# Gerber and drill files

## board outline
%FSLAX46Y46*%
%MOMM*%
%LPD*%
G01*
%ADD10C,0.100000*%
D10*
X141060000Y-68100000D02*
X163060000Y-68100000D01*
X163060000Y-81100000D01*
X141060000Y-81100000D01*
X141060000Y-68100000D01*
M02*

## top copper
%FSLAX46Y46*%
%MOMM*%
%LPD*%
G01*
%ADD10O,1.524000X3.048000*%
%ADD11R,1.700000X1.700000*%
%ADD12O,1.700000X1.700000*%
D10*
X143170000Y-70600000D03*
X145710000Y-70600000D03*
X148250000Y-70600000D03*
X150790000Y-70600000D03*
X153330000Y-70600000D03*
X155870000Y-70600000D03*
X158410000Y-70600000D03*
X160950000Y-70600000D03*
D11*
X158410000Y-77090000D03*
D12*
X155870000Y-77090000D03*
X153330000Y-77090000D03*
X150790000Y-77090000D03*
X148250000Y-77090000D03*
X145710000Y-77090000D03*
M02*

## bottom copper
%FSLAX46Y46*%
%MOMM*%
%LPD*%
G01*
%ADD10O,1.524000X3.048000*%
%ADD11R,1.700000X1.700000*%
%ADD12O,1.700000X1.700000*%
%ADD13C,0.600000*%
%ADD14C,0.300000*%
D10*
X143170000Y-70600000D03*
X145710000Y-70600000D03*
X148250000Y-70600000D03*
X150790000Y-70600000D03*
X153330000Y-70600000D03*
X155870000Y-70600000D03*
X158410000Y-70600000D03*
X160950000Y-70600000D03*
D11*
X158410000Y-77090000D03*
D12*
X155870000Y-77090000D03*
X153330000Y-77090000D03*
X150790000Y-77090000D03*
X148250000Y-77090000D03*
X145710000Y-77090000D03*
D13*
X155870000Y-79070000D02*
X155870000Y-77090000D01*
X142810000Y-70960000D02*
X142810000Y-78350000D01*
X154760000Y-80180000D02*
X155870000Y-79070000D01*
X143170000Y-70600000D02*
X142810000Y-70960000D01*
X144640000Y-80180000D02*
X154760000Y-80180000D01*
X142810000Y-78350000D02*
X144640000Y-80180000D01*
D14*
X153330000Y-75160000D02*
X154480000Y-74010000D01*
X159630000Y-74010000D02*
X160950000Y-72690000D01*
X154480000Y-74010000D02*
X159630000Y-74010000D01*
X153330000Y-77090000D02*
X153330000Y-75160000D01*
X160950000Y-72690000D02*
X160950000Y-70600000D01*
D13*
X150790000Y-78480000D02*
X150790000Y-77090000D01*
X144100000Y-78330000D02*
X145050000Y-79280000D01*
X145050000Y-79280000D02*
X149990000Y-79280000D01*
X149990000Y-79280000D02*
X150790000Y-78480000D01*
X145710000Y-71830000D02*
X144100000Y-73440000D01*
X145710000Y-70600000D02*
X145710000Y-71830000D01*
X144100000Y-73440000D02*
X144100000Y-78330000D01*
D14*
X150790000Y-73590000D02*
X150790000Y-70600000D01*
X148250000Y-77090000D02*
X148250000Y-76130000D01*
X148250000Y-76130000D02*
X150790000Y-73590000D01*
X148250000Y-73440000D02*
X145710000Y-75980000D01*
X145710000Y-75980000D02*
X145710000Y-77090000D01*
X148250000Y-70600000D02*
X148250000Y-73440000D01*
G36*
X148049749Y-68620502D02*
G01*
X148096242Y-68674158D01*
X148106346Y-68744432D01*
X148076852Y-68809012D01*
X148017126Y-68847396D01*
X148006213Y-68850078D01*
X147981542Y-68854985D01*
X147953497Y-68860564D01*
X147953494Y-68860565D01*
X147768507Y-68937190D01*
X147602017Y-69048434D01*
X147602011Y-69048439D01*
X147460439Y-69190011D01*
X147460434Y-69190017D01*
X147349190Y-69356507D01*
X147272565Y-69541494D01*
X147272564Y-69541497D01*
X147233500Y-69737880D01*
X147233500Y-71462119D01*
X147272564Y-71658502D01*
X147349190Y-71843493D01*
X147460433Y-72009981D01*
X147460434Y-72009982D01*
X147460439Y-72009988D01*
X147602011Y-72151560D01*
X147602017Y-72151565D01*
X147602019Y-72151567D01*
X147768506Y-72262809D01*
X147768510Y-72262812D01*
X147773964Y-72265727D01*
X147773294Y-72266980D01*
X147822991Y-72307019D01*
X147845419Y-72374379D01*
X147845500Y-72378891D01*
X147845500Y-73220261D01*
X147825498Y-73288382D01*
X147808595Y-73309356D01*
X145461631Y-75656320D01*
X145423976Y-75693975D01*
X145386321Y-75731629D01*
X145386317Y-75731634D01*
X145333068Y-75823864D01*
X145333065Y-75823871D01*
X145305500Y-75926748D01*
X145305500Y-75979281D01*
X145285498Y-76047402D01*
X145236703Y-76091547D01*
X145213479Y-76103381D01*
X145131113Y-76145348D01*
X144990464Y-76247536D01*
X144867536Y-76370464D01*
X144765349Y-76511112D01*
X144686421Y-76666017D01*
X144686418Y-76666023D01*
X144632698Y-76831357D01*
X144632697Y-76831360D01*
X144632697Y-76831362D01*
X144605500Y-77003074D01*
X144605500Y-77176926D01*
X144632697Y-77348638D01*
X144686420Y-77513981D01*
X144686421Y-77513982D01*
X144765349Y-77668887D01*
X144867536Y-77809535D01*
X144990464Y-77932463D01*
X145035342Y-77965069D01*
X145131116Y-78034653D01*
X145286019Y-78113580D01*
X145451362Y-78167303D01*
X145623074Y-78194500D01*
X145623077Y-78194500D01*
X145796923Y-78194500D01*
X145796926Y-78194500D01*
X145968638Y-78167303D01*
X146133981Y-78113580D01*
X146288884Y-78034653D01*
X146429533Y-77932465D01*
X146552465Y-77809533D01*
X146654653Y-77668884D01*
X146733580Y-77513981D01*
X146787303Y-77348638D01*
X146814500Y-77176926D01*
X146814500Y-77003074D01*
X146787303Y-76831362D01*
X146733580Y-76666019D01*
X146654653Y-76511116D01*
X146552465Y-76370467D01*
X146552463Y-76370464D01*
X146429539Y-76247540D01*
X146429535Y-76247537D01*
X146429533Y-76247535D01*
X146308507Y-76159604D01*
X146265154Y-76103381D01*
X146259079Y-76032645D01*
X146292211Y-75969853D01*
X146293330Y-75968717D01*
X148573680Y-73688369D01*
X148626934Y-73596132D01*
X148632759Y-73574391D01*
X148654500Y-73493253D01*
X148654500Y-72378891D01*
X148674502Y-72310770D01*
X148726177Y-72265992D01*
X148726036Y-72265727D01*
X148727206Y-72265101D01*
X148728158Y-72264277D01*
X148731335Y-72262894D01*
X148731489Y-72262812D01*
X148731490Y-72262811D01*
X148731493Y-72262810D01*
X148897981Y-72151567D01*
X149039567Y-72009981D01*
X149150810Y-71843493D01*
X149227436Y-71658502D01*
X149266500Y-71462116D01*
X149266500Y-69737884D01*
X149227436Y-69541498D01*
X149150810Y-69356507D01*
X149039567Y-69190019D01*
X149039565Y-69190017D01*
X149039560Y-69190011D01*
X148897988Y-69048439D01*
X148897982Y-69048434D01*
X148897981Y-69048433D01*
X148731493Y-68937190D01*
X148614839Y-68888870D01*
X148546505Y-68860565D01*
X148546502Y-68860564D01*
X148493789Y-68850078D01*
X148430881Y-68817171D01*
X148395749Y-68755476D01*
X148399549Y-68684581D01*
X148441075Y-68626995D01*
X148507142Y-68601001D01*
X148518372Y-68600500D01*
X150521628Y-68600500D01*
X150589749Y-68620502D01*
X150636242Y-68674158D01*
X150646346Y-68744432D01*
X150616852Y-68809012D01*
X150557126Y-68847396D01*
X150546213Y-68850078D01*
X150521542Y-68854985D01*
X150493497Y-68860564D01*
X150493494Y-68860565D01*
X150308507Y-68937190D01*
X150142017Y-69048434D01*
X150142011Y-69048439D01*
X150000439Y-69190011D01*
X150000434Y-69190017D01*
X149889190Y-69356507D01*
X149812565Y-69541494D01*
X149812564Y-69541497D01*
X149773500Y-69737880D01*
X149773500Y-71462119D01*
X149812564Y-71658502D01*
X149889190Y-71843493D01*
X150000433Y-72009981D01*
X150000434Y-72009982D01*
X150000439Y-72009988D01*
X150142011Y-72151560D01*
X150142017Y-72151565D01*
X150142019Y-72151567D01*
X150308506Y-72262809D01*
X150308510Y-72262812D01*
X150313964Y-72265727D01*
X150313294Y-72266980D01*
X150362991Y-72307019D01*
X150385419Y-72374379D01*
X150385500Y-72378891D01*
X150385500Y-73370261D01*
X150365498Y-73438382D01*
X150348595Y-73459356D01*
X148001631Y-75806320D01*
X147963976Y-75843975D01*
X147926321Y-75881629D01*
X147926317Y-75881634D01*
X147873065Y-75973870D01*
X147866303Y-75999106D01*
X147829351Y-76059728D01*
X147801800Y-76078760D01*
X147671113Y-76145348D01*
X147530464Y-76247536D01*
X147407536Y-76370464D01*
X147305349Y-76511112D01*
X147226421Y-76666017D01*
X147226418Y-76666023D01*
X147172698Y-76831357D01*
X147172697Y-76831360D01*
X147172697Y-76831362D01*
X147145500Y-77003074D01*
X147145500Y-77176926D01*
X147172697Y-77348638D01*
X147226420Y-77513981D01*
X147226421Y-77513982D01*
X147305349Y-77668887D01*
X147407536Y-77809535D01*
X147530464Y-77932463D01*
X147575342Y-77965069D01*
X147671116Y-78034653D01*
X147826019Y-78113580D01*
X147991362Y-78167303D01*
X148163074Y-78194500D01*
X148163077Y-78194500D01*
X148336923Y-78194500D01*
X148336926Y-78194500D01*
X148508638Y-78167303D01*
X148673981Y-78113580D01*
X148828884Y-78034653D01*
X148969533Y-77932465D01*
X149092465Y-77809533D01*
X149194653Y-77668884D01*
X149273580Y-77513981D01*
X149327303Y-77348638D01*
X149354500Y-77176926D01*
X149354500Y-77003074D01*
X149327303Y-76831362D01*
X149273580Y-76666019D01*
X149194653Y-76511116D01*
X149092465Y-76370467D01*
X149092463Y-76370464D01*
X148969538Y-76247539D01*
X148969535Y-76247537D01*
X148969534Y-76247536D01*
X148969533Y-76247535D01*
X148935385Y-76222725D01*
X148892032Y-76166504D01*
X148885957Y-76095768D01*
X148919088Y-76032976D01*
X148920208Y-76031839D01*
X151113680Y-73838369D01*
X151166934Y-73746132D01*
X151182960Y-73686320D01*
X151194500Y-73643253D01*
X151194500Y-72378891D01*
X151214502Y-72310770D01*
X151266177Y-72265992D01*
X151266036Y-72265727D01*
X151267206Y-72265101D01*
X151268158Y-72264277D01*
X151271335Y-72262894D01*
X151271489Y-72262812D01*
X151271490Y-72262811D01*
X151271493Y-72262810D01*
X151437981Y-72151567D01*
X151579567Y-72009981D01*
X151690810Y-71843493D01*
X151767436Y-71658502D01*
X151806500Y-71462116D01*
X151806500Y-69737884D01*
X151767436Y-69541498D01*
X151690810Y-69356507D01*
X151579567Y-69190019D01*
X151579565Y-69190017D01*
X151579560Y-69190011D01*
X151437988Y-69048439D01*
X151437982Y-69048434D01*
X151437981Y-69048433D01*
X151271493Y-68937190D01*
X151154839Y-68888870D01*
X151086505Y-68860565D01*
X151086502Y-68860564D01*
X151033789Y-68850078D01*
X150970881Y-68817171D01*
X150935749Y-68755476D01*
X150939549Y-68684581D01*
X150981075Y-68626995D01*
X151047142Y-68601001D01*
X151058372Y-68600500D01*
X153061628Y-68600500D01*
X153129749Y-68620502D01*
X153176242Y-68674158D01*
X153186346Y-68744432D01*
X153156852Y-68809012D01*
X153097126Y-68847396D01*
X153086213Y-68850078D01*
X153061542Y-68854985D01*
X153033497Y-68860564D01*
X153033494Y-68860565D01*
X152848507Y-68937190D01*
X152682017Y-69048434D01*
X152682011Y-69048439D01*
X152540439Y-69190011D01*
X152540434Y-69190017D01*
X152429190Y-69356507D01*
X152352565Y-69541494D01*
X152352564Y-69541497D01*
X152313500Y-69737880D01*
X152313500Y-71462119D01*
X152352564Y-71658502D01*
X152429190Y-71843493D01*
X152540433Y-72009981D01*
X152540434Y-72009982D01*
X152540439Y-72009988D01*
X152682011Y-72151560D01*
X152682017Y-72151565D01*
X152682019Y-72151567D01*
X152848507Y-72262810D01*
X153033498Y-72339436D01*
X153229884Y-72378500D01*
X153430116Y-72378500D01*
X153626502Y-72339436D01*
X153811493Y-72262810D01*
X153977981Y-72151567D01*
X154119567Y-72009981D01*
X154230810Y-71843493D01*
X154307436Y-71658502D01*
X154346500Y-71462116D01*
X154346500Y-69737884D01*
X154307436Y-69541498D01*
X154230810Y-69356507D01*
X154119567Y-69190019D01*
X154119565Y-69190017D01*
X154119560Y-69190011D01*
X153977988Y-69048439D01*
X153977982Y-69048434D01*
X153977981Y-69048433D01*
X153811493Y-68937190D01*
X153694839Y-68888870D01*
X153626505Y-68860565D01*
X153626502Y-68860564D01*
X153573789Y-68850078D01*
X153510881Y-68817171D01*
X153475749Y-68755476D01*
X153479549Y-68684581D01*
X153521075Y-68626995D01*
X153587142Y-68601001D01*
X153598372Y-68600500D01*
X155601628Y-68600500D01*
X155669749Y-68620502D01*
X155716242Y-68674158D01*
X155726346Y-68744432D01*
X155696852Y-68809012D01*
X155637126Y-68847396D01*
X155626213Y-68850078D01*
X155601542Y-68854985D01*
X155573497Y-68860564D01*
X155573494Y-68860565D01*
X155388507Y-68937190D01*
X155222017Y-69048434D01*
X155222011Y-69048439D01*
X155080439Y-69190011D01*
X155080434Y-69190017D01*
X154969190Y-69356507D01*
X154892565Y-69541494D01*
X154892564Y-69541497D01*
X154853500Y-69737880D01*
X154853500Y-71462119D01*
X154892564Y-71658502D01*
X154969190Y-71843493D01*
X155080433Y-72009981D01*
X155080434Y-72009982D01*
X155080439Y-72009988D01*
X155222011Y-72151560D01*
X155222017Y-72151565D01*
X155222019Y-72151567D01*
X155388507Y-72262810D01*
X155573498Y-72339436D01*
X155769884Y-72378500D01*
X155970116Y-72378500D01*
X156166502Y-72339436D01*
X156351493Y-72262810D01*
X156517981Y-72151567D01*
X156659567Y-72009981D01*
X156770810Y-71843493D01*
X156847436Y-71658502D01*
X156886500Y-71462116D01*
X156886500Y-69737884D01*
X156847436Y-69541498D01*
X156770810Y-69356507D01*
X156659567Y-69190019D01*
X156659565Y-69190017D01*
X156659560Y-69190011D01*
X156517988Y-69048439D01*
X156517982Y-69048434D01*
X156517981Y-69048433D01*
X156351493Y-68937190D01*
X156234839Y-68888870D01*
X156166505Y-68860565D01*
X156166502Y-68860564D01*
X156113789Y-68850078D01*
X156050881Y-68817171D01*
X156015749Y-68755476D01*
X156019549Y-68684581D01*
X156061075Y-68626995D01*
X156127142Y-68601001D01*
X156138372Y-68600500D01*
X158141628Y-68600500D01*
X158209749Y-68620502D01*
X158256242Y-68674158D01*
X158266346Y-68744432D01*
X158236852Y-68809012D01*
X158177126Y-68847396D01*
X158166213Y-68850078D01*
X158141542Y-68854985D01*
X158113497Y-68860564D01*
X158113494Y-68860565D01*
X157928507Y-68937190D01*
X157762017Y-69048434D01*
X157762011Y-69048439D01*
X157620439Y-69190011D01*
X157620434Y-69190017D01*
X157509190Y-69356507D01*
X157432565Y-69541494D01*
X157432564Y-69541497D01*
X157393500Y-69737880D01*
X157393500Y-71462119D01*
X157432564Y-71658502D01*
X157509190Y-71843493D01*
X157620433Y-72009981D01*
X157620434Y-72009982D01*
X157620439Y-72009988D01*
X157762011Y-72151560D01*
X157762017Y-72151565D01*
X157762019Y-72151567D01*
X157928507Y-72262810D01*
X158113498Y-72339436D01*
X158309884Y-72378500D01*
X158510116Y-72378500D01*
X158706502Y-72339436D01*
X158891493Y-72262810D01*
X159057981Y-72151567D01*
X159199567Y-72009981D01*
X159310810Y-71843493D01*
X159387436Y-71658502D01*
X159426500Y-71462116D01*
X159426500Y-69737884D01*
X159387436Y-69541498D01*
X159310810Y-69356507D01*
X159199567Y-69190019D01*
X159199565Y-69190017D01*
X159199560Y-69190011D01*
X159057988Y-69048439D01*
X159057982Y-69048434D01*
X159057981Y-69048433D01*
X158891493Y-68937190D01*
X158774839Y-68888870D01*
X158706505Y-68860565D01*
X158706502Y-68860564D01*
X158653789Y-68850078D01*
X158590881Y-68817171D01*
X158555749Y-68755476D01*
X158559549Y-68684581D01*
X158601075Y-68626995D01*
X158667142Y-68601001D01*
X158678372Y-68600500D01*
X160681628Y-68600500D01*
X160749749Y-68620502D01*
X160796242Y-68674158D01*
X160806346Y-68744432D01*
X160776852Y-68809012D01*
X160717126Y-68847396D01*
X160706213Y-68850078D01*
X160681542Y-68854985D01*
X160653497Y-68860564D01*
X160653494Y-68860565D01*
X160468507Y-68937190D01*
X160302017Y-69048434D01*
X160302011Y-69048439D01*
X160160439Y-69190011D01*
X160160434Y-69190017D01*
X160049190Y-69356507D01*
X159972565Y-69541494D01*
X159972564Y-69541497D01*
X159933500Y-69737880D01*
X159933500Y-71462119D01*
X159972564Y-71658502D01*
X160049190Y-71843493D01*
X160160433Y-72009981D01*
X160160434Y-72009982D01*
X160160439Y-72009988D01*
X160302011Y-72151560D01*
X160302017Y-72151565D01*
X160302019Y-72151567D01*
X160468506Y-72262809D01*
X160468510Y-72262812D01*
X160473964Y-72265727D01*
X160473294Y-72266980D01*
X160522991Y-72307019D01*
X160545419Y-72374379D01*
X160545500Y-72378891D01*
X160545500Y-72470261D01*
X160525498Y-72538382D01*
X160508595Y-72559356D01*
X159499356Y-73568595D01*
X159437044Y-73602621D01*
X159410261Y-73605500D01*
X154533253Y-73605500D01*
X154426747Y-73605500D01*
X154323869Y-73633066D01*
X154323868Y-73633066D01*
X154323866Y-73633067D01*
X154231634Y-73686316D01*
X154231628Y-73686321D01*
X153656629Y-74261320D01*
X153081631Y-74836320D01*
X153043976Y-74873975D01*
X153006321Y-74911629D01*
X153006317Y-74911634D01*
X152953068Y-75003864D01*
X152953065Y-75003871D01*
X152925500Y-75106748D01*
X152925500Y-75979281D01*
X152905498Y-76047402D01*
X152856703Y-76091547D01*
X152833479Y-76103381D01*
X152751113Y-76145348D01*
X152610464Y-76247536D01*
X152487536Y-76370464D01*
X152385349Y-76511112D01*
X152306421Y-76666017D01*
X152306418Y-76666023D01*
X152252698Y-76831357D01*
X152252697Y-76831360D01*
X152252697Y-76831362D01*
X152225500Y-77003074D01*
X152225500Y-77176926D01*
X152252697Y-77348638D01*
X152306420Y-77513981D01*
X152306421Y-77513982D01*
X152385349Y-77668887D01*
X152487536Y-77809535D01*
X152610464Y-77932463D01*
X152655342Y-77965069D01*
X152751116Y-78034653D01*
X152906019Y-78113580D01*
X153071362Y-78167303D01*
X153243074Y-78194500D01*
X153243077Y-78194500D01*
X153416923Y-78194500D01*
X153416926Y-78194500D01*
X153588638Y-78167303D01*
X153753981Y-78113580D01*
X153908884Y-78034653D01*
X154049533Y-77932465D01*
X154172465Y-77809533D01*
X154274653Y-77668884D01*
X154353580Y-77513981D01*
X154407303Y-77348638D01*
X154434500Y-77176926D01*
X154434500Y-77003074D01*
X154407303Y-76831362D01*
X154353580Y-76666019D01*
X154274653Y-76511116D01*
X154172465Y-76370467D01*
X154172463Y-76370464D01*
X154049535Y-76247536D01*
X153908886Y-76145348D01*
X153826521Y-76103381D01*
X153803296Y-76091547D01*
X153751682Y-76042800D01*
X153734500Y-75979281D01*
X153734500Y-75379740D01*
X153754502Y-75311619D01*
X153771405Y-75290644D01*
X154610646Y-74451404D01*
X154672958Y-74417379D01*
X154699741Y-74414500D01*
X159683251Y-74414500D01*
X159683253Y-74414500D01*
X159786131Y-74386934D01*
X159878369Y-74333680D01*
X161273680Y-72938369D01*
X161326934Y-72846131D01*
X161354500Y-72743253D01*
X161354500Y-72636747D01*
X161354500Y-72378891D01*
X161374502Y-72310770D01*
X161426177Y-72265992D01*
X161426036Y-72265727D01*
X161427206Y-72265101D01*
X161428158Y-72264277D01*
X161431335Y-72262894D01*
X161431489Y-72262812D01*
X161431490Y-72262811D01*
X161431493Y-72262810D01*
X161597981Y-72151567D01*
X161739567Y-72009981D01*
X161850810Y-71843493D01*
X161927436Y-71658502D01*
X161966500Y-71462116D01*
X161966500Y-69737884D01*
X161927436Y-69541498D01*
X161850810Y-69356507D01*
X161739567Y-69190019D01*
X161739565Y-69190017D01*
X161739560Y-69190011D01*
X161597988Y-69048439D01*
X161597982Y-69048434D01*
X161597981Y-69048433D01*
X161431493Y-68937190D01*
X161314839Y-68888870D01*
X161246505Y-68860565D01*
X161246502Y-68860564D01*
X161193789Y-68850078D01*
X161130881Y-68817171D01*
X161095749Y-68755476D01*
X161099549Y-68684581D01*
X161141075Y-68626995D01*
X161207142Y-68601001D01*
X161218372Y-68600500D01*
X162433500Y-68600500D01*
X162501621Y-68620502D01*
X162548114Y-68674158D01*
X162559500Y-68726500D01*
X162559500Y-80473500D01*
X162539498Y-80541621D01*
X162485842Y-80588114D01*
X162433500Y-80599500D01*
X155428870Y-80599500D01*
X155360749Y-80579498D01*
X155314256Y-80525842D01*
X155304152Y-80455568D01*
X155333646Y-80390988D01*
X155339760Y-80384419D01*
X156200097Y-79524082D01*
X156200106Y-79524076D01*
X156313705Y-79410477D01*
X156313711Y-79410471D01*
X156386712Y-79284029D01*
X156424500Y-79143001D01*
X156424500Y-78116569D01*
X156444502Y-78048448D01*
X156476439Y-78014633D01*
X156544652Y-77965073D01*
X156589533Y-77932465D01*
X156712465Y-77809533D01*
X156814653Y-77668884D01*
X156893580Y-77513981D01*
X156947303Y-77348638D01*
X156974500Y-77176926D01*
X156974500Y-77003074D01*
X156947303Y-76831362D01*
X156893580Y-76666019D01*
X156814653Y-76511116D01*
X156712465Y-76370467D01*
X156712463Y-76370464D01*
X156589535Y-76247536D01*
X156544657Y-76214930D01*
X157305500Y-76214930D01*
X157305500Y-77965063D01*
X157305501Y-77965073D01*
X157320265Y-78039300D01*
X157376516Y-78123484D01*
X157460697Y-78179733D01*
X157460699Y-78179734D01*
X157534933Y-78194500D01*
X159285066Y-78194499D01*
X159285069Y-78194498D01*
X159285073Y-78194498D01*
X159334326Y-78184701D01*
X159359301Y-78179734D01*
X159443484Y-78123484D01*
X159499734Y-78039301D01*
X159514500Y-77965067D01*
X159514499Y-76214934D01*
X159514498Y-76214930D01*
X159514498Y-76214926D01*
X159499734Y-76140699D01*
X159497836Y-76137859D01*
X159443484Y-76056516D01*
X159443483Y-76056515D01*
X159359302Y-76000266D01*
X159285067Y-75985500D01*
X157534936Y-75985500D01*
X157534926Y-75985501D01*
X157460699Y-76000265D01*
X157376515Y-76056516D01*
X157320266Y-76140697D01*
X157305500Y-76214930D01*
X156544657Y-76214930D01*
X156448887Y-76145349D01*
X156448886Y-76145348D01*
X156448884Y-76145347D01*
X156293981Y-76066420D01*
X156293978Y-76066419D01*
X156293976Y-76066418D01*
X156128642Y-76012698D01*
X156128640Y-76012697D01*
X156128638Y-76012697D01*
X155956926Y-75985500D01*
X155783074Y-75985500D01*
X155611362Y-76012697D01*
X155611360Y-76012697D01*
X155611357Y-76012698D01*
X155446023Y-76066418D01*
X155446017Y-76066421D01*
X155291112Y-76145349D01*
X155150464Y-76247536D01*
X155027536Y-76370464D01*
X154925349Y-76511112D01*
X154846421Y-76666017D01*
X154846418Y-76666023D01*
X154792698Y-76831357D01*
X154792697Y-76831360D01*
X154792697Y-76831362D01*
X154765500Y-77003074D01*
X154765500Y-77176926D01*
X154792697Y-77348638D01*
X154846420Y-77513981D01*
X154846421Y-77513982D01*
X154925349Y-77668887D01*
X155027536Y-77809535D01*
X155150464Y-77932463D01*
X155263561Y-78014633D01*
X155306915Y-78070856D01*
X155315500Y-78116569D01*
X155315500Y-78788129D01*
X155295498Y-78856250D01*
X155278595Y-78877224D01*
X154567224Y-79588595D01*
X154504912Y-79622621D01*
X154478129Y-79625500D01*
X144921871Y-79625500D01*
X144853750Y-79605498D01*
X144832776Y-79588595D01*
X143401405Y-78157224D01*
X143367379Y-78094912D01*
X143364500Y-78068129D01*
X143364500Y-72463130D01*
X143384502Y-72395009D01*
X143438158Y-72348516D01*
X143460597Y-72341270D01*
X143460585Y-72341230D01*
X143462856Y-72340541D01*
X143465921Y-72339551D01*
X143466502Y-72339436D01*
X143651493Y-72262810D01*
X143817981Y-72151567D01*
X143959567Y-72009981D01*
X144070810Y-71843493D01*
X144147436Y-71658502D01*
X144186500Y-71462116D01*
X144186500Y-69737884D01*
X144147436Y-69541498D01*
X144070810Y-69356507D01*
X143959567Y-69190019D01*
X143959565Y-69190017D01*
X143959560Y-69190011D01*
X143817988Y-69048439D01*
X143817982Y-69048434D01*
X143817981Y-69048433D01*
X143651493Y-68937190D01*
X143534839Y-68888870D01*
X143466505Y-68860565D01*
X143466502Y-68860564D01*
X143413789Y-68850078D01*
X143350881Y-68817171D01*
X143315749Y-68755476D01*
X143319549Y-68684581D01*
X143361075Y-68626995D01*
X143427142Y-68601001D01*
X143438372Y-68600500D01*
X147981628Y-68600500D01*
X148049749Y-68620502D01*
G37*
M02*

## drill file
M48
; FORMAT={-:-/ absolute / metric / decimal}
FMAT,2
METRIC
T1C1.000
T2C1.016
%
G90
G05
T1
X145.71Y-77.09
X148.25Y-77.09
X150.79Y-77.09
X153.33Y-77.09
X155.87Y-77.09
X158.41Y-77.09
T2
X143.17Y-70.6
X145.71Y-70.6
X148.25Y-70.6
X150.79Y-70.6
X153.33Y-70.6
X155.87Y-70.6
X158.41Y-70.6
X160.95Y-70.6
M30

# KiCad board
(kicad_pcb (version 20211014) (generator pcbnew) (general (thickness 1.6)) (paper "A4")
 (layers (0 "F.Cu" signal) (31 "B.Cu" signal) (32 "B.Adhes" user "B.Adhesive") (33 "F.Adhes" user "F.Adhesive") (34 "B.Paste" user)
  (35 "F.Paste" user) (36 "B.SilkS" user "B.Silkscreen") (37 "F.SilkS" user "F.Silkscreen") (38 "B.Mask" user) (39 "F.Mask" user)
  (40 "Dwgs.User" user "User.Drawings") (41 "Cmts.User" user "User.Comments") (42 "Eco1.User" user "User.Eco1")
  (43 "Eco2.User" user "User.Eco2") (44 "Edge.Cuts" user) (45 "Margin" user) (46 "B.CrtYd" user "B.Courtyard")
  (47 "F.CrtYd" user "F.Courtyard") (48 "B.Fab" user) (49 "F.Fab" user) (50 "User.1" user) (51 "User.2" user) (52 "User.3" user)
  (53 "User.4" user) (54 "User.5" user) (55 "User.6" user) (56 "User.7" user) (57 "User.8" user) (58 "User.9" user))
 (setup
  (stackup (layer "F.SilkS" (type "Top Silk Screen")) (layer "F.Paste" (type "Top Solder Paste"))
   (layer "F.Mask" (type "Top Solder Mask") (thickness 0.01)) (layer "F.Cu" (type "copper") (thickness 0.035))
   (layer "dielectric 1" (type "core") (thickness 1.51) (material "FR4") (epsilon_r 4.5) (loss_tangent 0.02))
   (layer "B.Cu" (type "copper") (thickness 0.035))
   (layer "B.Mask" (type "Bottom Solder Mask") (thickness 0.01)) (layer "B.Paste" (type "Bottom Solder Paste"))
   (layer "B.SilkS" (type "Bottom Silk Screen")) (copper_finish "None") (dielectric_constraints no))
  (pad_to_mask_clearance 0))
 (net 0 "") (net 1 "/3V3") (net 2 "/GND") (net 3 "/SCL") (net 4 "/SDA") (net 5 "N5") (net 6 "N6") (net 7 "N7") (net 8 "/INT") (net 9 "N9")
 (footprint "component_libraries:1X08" (layer "F.Cu") (at 152.06 70.6)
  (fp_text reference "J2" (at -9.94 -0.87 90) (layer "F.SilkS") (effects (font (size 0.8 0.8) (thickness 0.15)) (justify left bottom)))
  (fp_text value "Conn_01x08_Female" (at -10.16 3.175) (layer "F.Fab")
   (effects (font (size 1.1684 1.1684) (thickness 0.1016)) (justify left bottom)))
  (pad "1" thru_hole oval (at -8.89 0 90) (size 3.048 1.524) (drill 1.016) (layers *.Cu *.Mask) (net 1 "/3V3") (solder_mask_margin 0.1016))
  (pad "2" thru_hole oval (at -6.35 0 90) (size 3.048 1.524) (drill 1.016) (layers *.Cu *.Mask) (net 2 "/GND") (solder_mask_margin 0.1016))
  (pad "3" thru_hole oval (at -3.81 0 90) (size 3.048 1.524) (drill 1.016) (layers *.Cu *.Mask) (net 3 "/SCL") (solder_mask_margin 0.1016))
  (pad "4" thru_hole oval (at -1.27 0 90) (size 3.048 1.524) (drill 1.016) (layers *.Cu *.Mask) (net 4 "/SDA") (solder_mask_margin 0.1016))
  (pad "5" thru_hole oval (at 1.27 0 90) (size 3.048 1.524) (drill 1.016) (layers *.Cu *.Mask) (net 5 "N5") (solder_mask_margin 0.1016))
  (pad "6" thru_hole oval (at 3.81 0 90) (size 3.048 1.524) (drill 1.016) (layers *.Cu *.Mask) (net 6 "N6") (solder_mask_margin 0.1016))
  (pad "7" thru_hole oval (at 6.35 0 90) (size 3.048 1.524) (drill 1.016) (layers *.Cu *.Mask) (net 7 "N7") (solder_mask_margin 0.1016))
  (pad "8" thru_hole oval (at 8.89 0 90) (size 3.048 1.524) (drill 1.016) (layers *.Cu *.Mask) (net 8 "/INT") (solder_mask_margin 0.1016)))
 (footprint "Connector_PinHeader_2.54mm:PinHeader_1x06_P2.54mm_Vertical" (layer "F.Cu") (at 158.41 77.09 -90)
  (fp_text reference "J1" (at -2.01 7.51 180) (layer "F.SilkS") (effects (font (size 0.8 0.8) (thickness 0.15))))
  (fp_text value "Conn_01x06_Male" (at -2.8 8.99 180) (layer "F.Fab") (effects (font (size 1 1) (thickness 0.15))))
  (pad "1" thru_hole rect locked (at 0 0 270) (size 1.7 1.7) (drill 1) (layers *.Cu *.Mask) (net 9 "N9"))
  (pad "2" thru_hole oval locked (at 0 2.54 270) (size 1.7 1.7) (drill 1) (layers *.Cu *.Mask) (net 1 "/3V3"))
  (pad "3" thru_hole oval locked (at 0 5.08 270) (size 1.7 1.7) (drill 1) (layers *.Cu *.Mask) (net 8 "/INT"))
  (pad "4" thru_hole oval locked (at 0 7.62 270) (size 1.7 1.7) (drill 1) (layers *.Cu *.Mask) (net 2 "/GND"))
  (pad "5" thru_hole oval locked (at 0 10.16 270) (size 1.7 1.7) (drill 1) (layers *.Cu *.Mask) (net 4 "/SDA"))
  (pad "6" thru_hole oval locked (at 0 12.7 270) (size 1.7 1.7) (drill 1) (layers *.Cu *.Mask) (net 3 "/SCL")))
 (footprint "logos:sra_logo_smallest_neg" (layer "F.Cu") (at 142.31 77.09 90)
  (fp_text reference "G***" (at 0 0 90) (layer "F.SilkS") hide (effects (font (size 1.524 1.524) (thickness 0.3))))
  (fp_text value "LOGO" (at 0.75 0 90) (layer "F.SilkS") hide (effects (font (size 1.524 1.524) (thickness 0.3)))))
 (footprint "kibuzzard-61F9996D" (layer "F.Cu") (at 162.13 77.32 90)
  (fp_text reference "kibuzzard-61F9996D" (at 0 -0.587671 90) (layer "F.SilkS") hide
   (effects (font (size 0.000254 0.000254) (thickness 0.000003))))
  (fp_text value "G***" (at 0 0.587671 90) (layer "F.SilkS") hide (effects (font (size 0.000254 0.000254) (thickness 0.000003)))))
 (gr_rect (start 141.06 68.1) (end 163.06 81.1) (layer "Edge.Cuts") (width 0.1) (fill none))
 (segment (start 155.87 79.07) (end 155.87 77.09) (width 0.6) (layer "B.Cu") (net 1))
 (segment (start 142.81 70.96) (end 142.81 78.35) (width 0.6) (layer "B.Cu") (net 1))
 (segment (start 154.76 80.18) (end 155.87 79.07) (width 0.6) (layer "B.Cu") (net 1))
 (segment (start 143.17 70.6) (end 142.81 70.96) (width 0.6) (layer "B.Cu") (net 1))
 (segment (start 144.64 80.18) (end 154.76 80.18) (width 0.6) (layer "B.Cu") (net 1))
 (segment (start 142.81 78.35) (end 144.64 80.18) (width 0.6) (layer "B.Cu") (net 1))
 (segment (start 153.33 75.16) (end 154.48 74.01) (width 0.3) (layer "B.Cu") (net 8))
 (segment (start 159.63 74.01) (end 160.95 72.69) (width 0.3) (layer "B.Cu") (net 8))
 (segment (start 154.48 74.01) (end 159.63 74.01) (width 0.3) (layer "B.Cu") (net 8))
 (segment (start 153.33 77.09) (end 153.33 75.16) (width 0.3) (layer "B.Cu") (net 8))
 (segment (start 160.95 72.69) (end 160.95 70.6) (width 0.3) (layer "B.Cu") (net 8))
 (segment (start 150.79 78.48) (end 150.79 77.09) (width 0.6) (layer "B.Cu") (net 2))
 (segment (start 144.1 78.33) (end 145.05 79.28) (width 0.6) (layer "B.Cu") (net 2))
 (segment (start 145.05 79.28) (end 149.99 79.28) (width 0.6) (layer "B.Cu") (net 2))
 (segment (start 149.99 79.28) (end 150.79 78.48) (width 0.6) (layer "B.Cu") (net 2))
 (segment (start 145.71 71.83) (end 144.1 73.44) (width 0.6) (layer "B.Cu") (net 2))
 (segment (start 145.71 70.6) (end 145.71 71.83) (width 0.6) (layer "B.Cu") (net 2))
 (segment (start 144.1 73.44) (end 144.1 78.33) (width 0.6) (layer "B.Cu") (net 2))
 (segment (start 150.79 73.59) (end 150.79 70.6) (width 0.3) (layer "B.Cu") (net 4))
 (segment (start 148.25 77.09) (end 148.25 76.13) (width 0.3) (layer "B.Cu") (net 4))
 (segment (start 148.25 76.13) (end 150.79 73.59) (width 0.3) (layer "B.Cu") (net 4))
 (segment (start 148.25 73.44) (end 145.71 75.98) (width 0.3) (layer "B.Cu") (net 3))
 (segment (start 145.71 75.98) (end 145.71 77.09) (width 0.3) (layer "B.Cu") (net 3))
 (segment (start 148.25 70.6) (end 148.25 73.44) (width 0.3) (layer "B.Cu") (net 3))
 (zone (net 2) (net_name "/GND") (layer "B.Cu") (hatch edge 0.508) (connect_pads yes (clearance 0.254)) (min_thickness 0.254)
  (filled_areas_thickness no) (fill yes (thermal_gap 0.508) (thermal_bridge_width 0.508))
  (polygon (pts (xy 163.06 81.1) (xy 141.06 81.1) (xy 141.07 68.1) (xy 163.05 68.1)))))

